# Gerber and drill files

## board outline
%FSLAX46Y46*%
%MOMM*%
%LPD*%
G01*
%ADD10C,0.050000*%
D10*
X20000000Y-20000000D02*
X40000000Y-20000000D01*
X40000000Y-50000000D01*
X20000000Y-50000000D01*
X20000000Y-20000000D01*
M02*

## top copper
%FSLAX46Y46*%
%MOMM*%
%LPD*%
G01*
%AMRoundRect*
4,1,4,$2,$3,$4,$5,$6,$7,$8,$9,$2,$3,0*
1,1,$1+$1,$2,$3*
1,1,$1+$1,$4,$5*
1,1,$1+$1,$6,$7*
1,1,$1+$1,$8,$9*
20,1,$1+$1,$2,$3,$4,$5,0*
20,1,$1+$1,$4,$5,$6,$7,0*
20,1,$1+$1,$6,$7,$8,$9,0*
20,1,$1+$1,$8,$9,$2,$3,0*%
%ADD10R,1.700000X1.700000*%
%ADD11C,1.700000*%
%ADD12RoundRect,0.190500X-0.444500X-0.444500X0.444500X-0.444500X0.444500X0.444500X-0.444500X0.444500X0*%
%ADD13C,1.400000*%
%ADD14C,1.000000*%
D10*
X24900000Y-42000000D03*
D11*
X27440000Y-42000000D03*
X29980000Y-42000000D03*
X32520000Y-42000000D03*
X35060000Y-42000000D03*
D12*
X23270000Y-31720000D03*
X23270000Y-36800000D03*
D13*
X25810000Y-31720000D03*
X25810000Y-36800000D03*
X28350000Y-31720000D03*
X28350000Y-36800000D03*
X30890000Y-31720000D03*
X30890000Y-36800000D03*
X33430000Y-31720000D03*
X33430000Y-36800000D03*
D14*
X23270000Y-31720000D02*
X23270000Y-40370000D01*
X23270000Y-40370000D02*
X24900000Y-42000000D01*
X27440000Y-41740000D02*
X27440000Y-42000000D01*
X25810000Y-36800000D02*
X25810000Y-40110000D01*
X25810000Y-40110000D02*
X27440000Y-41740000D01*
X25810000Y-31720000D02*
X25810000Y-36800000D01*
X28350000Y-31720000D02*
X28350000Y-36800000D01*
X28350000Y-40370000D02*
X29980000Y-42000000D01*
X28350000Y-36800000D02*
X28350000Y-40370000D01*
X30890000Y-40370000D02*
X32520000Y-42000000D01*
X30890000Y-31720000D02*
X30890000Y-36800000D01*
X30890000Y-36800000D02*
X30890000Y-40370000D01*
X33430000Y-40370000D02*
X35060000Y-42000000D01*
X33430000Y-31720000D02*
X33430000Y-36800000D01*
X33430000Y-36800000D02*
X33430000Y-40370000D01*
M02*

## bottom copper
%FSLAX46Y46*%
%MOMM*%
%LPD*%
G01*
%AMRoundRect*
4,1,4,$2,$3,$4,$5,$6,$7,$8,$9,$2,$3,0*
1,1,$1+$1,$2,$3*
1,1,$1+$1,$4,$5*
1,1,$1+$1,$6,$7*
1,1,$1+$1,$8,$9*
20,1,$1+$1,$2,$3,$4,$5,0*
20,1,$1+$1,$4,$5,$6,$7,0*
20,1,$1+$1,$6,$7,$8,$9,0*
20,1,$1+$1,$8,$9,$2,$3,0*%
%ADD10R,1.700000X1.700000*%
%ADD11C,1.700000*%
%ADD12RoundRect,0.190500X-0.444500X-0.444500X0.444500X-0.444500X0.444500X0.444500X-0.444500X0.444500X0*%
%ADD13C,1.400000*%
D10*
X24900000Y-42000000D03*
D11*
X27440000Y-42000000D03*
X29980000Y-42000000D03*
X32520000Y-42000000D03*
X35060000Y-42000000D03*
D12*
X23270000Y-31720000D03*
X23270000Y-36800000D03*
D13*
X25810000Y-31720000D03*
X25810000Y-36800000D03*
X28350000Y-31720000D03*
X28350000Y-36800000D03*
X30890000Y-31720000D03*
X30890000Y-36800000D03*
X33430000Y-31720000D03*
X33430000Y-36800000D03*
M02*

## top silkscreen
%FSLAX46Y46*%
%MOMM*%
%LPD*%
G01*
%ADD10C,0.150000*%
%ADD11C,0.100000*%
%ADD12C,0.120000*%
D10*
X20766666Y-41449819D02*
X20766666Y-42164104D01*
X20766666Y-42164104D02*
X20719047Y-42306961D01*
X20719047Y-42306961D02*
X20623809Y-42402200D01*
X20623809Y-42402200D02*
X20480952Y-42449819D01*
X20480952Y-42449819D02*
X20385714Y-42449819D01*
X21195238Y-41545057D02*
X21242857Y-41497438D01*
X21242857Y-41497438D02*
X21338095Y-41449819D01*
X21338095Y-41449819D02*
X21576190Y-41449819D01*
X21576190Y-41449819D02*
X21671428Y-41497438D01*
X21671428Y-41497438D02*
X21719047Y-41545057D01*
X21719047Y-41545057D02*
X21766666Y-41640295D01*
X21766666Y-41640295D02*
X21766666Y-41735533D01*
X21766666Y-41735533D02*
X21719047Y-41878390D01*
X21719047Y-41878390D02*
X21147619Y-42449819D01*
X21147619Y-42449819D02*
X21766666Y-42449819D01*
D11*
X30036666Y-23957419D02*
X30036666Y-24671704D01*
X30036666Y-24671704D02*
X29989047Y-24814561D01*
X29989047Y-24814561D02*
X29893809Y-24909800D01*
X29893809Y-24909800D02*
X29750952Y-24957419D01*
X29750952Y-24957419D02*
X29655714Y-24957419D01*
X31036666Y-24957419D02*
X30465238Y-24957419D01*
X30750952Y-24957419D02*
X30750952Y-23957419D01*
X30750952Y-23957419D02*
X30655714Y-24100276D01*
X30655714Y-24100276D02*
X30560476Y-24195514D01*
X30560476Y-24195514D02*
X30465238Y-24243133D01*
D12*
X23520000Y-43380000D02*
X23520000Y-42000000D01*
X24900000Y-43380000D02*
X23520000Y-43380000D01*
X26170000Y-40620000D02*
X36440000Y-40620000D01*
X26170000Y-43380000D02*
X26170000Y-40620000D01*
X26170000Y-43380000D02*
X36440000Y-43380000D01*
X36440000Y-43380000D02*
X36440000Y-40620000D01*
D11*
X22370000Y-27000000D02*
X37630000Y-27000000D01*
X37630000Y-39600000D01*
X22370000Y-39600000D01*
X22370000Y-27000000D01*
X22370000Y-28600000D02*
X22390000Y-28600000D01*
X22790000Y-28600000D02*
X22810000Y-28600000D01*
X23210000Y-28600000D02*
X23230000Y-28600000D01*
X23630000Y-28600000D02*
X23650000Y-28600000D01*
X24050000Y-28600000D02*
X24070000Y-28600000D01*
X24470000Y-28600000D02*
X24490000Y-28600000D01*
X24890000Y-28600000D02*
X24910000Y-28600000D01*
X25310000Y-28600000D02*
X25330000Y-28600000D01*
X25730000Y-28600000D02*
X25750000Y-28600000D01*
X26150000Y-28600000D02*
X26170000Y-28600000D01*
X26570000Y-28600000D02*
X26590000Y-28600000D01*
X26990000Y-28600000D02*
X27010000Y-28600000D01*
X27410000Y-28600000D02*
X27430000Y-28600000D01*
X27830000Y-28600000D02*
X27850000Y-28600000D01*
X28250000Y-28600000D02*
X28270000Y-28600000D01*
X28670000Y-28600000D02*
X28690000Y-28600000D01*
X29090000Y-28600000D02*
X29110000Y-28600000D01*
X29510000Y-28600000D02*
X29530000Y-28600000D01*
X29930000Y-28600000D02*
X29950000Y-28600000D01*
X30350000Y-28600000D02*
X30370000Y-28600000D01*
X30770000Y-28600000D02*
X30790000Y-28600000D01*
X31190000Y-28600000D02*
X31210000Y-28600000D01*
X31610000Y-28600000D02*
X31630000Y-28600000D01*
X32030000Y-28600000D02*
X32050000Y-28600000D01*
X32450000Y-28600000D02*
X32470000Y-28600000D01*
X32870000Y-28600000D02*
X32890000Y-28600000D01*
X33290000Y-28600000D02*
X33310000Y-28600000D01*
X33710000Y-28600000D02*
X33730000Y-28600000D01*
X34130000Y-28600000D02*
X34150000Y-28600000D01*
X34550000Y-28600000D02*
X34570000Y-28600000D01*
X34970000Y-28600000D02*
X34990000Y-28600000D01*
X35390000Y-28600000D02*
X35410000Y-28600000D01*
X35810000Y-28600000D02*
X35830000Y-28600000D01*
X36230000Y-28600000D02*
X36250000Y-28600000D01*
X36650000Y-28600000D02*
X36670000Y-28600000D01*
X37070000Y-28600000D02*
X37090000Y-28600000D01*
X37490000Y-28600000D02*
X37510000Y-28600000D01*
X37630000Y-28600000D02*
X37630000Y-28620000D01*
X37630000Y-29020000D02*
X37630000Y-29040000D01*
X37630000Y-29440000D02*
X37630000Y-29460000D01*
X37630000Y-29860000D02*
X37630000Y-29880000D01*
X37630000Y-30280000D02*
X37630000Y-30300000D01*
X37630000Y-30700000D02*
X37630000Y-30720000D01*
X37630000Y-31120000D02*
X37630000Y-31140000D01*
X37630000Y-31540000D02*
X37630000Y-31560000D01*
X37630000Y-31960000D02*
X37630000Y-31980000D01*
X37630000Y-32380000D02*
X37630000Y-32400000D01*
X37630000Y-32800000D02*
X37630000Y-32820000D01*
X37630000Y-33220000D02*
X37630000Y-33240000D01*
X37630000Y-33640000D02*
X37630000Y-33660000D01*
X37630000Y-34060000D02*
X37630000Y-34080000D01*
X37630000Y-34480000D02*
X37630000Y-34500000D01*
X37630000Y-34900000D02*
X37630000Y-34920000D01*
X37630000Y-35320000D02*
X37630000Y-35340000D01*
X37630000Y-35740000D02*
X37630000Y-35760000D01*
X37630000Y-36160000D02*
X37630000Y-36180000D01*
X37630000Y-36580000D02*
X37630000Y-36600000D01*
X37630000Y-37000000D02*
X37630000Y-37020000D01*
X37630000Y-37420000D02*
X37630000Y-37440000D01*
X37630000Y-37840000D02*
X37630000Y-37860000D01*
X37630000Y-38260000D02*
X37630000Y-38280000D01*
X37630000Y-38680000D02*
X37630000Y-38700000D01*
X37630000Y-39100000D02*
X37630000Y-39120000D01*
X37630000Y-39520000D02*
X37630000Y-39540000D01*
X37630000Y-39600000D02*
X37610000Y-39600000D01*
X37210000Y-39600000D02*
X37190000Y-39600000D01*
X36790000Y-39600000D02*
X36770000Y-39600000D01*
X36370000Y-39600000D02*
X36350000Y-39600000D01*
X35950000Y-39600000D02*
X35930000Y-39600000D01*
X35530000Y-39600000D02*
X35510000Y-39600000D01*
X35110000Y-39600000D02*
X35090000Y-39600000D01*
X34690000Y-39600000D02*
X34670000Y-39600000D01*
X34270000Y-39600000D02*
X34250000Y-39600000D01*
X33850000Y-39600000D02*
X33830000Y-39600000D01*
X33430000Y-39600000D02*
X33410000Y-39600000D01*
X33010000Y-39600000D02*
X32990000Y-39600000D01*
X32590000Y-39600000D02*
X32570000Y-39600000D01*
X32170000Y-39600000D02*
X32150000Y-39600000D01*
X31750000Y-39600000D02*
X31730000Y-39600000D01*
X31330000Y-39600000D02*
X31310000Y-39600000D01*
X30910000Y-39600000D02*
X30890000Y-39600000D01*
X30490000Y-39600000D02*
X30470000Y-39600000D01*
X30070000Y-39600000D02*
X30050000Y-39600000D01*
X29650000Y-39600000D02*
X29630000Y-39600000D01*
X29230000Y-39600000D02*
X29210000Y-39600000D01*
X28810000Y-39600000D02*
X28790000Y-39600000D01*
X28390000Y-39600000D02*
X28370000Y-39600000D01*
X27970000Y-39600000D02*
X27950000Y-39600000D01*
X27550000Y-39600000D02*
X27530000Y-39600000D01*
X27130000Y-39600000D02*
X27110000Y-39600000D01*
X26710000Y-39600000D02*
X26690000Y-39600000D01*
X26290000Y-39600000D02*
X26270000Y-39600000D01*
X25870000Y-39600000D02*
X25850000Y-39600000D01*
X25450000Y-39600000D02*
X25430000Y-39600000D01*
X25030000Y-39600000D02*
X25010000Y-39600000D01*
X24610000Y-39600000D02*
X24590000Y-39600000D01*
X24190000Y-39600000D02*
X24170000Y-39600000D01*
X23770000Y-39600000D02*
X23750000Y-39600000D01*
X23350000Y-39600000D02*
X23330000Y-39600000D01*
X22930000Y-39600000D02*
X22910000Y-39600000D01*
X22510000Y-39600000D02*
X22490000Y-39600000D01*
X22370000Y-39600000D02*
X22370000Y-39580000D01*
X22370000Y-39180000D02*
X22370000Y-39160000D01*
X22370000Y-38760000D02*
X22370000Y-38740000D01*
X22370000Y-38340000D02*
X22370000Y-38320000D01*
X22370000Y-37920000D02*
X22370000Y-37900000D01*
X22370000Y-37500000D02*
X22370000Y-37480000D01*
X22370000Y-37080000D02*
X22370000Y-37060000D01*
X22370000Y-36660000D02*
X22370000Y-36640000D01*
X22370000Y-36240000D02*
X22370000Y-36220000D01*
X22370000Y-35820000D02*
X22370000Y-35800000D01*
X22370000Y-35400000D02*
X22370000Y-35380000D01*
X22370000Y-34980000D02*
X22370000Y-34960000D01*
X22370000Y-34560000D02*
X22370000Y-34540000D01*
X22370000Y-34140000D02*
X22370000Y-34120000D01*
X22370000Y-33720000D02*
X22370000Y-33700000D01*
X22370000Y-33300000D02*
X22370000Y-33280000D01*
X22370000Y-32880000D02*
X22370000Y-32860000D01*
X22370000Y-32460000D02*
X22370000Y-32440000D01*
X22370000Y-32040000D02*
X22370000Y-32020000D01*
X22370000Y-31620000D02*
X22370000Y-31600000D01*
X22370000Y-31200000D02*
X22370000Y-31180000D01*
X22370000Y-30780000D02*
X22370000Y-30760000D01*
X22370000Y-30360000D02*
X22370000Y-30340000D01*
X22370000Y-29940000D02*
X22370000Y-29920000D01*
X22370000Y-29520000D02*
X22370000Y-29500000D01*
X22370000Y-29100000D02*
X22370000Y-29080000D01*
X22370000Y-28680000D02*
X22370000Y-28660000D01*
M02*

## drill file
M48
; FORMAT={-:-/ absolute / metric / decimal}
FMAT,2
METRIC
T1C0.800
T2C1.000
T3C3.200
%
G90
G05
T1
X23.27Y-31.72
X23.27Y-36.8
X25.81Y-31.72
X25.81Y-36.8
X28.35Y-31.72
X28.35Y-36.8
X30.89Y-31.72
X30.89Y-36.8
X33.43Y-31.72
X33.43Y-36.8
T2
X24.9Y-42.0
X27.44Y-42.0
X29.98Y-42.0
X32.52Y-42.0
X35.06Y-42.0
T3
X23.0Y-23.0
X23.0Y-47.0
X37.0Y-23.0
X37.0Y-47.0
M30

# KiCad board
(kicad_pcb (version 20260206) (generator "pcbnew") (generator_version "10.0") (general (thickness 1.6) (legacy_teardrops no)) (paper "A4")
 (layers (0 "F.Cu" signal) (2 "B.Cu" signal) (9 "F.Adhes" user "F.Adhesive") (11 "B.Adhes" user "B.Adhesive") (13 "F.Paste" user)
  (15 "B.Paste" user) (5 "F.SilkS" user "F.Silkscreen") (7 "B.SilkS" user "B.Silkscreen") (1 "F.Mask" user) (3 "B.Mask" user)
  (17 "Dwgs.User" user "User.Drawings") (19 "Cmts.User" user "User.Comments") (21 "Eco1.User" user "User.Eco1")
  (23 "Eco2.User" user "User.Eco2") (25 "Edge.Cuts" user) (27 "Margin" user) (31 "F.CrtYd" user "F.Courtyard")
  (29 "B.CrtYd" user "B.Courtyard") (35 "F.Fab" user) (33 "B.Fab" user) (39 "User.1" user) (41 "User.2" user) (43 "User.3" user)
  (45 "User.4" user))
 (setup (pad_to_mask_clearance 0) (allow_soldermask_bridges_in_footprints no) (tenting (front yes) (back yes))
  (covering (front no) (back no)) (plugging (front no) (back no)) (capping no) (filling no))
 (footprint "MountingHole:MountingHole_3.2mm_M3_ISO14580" (layer "F.Cu") (at 23 47)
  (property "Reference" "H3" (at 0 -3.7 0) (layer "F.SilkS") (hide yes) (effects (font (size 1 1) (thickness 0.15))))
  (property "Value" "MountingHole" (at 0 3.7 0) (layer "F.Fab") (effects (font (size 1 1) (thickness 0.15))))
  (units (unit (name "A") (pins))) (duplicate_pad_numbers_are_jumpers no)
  (pad "" np_thru_hole circle (at 0 0) (size 3.2 3.2) (drill 3.2) (layers "*.Cu" "*.Mask")))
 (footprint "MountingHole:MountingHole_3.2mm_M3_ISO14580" (layer "F.Cu") (at 37 23)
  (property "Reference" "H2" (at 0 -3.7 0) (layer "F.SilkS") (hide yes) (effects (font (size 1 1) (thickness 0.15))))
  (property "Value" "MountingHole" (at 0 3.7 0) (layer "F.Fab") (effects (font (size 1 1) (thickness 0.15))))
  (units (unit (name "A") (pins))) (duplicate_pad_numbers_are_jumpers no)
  (pad "" np_thru_hole circle (at 0 0) (size 3.2 3.2) (drill 3.2) (layers "*.Cu" "*.Mask")))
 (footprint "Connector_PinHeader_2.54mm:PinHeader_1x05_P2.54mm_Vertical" (layer "F.Cu") (at 24.9 42 90)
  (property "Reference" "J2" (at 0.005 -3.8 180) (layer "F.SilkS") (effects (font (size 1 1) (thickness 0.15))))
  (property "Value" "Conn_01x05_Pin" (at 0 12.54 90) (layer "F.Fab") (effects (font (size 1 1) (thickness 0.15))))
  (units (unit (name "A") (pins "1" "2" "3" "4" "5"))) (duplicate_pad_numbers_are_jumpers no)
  (fp_line (start -1.38 -1.38) (end 0 -1.38) (stroke (width 0.12) (type solid)) (layer "F.SilkS"))
  (fp_line (start -1.38 0) (end -1.38 -1.38) (stroke (width 0.12) (type solid)) (layer "F.SilkS"))
  (fp_line (start 1.38 1.27) (end 1.38 11.54) (stroke (width 0.12) (type solid)) (layer "F.SilkS"))
  (fp_line (start -1.38 1.27) (end 1.38 1.27) (stroke (width 0.12) (type solid)) (layer "F.SilkS"))
  (fp_line (start -1.38 1.27) (end -1.38 11.54) (stroke (width 0.12) (type solid)) (layer "F.SilkS"))
  (fp_line (start -1.38 11.54) (end 1.38 11.54) (stroke (width 0.12) (type solid)) (layer "F.SilkS"))
  (pad "1" thru_hole rect (at 0 0 90) (size 1.7 1.7) (drill 1) (layers "*.Cu" "*.Mask") (remove_unused_layers no) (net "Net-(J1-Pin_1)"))
  (pad "2" thru_hole circle (at 0 2.54 90) (size 1.7 1.7) (drill 1) (layers "*.Cu" "*.Mask") (remove_unused_layers no)
   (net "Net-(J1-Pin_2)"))
  (pad "3" thru_hole circle (at 0 5.08 90) (size 1.7 1.7) (drill 1) (layers "*.Cu" "*.Mask") (remove_unused_layers no)
   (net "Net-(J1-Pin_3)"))
  (pad "4" thru_hole circle (at 0 7.62 90) (size 1.7 1.7) (drill 1) (layers "*.Cu" "*.Mask") (remove_unused_layers no)
   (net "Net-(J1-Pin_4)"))
  (pad "5" thru_hole circle (at 0 10.16 90) (size 1.7 1.7) (drill 1) (layers "*.Cu" "*.Mask") (remove_unused_layers no)
   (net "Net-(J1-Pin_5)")))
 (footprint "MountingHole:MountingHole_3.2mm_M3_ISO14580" (layer "F.Cu") (at 23 23)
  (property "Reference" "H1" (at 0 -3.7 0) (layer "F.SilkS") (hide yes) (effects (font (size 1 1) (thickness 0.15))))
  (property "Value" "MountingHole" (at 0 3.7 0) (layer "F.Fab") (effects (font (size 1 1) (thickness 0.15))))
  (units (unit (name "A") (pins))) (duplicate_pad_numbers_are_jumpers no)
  (pad "" np_thru_hole circle (at 0 0) (size 3.2 3.2) (drill 3.2) (layers "*.Cu" "*.Mask")))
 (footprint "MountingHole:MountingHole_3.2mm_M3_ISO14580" (layer "F.Cu") (at 37 47)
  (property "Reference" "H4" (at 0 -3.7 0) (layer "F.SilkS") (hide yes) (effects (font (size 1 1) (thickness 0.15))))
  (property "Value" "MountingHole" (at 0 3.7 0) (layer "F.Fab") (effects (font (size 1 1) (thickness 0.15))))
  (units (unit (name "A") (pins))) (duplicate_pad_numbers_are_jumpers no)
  (pad "" np_thru_hole circle (at 0 0) (size 3.2 3.2) (drill 3.2) (layers "*.Cu" "*.Mask")))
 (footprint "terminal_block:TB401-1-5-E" (layer "F.Cu") (at 22.37 27)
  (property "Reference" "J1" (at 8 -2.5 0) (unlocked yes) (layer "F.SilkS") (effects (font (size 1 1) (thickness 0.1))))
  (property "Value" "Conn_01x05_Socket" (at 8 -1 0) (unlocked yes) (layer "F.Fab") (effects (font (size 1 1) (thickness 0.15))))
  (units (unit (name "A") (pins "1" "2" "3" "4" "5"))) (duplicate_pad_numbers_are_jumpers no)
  (fp_rect (start 0 0) (end 15.26 12.6) (stroke (width 0.1) (type solid)) (fill no) (layer "F.SilkS"))
  (fp_rect (start 0 1.6) (end 15.26 12.6) (stroke (width 0.1) (type dot)) (fill no) (layer "F.SilkS"))
  (pad "1" thru_hole roundrect (at 0.9 4.72) (size 1.27 1.27) (drill 0.8) (layers "*.Cu" "*.Mask" "Eco2.User") (remove_unused_layers no)
   (roundrect_rratio 0.15) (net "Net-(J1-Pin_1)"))
  (pad "1" thru_hole roundrect (at 0.9 9.8) (size 1.27 1.27) (drill 0.8) (layers "*.Cu" "*.Mask" "Eco2.User") (remove_unused_layers no)
   (roundrect_rratio 0.15) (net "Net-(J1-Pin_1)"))
  (pad "2" thru_hole circle (at 3.44 4.72) (size 1.4 1.4) (drill 0.8) (layers "*.Cu" "*.Mask") (remove_unused_layers no)
   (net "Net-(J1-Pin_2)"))
  (pad "2" thru_hole circle (at 3.44 9.8) (size 1.4 1.4) (drill 0.8) (layers "*.Cu" "*.Mask") (remove_unused_layers no)
   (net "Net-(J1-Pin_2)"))
  (pad "3" thru_hole circle (at 5.98 4.72) (size 1.4 1.4) (drill 0.8) (layers "*.Cu" "*.Mask") (remove_unused_layers no)
   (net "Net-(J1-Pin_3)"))
  (pad "3" thru_hole circle (at 5.98 9.8) (size 1.4 1.4) (drill 0.8) (layers "*.Cu" "*.Mask") (remove_unused_layers no)
   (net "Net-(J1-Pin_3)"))
  (pad "4" thru_hole circle (at 8.52 4.72) (size 1.4 1.4) (drill 0.8) (layers "*.Cu" "*.Mask") (remove_unused_layers no)
   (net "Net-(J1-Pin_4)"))
  (pad "4" thru_hole circle (at 8.52 9.8) (size 1.4 1.4) (drill 0.8) (layers "*.Cu" "*.Mask") (remove_unused_layers no)
   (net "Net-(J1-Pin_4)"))
  (pad "5" thru_hole circle (at 11.06 4.72) (size 1.4 1.4) (drill 0.8) (layers "*.Cu" "*.Mask") (remove_unused_layers no)
   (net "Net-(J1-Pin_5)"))
  (pad "5" thru_hole circle (at 11.06 9.8) (size 1.4 1.4) (drill 0.8) (layers "*.Cu" "*.Mask") (remove_unused_layers no)
   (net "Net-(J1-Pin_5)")))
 (gr_rect (start 20 20) (end 40 50) (stroke (width 0.05) (type solid)) (fill no) (layer "Edge.Cuts"))
 (segment (start 23.27 31.72) (end 23.27 40.37) (width 1) (layer "F.Cu") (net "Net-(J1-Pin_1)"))
 (segment (start 23.27 40.37) (end 24.9 42) (width 1) (layer "F.Cu") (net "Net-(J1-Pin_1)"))
 (segment (start 27.44 41.74) (end 27.44 42) (width 1) (layer "F.Cu") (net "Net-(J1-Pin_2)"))
 (segment (start 25.81 36.8) (end 25.81 40.11) (width 1) (layer "F.Cu") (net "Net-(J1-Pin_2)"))
 (segment (start 25.81 40.11) (end 27.44 41.74) (width 1) (layer "F.Cu") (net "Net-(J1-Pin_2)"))
 (segment (start 25.81 31.72) (end 25.81 36.8) (width 1) (layer "F.Cu") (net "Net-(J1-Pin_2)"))
 (segment (start 28.35 31.72) (end 28.35 36.8) (width 1) (layer "F.Cu") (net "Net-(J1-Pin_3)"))
 (segment (start 28.35 40.37) (end 29.98 42) (width 1) (layer "F.Cu") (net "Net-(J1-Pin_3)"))
 (segment (start 28.35 36.8) (end 28.35 40.37) (width 1) (layer "F.Cu") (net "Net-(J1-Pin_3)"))
 (segment (start 30.89 40.37) (end 32.52 42) (width 1) (layer "F.Cu") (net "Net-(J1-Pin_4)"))
 (segment (start 30.89 31.72) (end 30.89 36.8) (width 1) (layer "F.Cu") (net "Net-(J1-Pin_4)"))
 (segment (start 30.89 36.8) (end 30.89 40.37) (width 1) (layer "F.Cu") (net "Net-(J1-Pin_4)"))
 (segment (start 33.43 40.37) (end 35.06 42) (width 1) (layer "F.Cu") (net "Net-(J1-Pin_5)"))
 (segment (start 33.43 31.72) (end 33.43 36.8) (width 1) (layer "F.Cu") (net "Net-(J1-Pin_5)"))
 (segment (start 33.43 36.8) (end 33.43 40.37) (width 1) (layer "F.Cu") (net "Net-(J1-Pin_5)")))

